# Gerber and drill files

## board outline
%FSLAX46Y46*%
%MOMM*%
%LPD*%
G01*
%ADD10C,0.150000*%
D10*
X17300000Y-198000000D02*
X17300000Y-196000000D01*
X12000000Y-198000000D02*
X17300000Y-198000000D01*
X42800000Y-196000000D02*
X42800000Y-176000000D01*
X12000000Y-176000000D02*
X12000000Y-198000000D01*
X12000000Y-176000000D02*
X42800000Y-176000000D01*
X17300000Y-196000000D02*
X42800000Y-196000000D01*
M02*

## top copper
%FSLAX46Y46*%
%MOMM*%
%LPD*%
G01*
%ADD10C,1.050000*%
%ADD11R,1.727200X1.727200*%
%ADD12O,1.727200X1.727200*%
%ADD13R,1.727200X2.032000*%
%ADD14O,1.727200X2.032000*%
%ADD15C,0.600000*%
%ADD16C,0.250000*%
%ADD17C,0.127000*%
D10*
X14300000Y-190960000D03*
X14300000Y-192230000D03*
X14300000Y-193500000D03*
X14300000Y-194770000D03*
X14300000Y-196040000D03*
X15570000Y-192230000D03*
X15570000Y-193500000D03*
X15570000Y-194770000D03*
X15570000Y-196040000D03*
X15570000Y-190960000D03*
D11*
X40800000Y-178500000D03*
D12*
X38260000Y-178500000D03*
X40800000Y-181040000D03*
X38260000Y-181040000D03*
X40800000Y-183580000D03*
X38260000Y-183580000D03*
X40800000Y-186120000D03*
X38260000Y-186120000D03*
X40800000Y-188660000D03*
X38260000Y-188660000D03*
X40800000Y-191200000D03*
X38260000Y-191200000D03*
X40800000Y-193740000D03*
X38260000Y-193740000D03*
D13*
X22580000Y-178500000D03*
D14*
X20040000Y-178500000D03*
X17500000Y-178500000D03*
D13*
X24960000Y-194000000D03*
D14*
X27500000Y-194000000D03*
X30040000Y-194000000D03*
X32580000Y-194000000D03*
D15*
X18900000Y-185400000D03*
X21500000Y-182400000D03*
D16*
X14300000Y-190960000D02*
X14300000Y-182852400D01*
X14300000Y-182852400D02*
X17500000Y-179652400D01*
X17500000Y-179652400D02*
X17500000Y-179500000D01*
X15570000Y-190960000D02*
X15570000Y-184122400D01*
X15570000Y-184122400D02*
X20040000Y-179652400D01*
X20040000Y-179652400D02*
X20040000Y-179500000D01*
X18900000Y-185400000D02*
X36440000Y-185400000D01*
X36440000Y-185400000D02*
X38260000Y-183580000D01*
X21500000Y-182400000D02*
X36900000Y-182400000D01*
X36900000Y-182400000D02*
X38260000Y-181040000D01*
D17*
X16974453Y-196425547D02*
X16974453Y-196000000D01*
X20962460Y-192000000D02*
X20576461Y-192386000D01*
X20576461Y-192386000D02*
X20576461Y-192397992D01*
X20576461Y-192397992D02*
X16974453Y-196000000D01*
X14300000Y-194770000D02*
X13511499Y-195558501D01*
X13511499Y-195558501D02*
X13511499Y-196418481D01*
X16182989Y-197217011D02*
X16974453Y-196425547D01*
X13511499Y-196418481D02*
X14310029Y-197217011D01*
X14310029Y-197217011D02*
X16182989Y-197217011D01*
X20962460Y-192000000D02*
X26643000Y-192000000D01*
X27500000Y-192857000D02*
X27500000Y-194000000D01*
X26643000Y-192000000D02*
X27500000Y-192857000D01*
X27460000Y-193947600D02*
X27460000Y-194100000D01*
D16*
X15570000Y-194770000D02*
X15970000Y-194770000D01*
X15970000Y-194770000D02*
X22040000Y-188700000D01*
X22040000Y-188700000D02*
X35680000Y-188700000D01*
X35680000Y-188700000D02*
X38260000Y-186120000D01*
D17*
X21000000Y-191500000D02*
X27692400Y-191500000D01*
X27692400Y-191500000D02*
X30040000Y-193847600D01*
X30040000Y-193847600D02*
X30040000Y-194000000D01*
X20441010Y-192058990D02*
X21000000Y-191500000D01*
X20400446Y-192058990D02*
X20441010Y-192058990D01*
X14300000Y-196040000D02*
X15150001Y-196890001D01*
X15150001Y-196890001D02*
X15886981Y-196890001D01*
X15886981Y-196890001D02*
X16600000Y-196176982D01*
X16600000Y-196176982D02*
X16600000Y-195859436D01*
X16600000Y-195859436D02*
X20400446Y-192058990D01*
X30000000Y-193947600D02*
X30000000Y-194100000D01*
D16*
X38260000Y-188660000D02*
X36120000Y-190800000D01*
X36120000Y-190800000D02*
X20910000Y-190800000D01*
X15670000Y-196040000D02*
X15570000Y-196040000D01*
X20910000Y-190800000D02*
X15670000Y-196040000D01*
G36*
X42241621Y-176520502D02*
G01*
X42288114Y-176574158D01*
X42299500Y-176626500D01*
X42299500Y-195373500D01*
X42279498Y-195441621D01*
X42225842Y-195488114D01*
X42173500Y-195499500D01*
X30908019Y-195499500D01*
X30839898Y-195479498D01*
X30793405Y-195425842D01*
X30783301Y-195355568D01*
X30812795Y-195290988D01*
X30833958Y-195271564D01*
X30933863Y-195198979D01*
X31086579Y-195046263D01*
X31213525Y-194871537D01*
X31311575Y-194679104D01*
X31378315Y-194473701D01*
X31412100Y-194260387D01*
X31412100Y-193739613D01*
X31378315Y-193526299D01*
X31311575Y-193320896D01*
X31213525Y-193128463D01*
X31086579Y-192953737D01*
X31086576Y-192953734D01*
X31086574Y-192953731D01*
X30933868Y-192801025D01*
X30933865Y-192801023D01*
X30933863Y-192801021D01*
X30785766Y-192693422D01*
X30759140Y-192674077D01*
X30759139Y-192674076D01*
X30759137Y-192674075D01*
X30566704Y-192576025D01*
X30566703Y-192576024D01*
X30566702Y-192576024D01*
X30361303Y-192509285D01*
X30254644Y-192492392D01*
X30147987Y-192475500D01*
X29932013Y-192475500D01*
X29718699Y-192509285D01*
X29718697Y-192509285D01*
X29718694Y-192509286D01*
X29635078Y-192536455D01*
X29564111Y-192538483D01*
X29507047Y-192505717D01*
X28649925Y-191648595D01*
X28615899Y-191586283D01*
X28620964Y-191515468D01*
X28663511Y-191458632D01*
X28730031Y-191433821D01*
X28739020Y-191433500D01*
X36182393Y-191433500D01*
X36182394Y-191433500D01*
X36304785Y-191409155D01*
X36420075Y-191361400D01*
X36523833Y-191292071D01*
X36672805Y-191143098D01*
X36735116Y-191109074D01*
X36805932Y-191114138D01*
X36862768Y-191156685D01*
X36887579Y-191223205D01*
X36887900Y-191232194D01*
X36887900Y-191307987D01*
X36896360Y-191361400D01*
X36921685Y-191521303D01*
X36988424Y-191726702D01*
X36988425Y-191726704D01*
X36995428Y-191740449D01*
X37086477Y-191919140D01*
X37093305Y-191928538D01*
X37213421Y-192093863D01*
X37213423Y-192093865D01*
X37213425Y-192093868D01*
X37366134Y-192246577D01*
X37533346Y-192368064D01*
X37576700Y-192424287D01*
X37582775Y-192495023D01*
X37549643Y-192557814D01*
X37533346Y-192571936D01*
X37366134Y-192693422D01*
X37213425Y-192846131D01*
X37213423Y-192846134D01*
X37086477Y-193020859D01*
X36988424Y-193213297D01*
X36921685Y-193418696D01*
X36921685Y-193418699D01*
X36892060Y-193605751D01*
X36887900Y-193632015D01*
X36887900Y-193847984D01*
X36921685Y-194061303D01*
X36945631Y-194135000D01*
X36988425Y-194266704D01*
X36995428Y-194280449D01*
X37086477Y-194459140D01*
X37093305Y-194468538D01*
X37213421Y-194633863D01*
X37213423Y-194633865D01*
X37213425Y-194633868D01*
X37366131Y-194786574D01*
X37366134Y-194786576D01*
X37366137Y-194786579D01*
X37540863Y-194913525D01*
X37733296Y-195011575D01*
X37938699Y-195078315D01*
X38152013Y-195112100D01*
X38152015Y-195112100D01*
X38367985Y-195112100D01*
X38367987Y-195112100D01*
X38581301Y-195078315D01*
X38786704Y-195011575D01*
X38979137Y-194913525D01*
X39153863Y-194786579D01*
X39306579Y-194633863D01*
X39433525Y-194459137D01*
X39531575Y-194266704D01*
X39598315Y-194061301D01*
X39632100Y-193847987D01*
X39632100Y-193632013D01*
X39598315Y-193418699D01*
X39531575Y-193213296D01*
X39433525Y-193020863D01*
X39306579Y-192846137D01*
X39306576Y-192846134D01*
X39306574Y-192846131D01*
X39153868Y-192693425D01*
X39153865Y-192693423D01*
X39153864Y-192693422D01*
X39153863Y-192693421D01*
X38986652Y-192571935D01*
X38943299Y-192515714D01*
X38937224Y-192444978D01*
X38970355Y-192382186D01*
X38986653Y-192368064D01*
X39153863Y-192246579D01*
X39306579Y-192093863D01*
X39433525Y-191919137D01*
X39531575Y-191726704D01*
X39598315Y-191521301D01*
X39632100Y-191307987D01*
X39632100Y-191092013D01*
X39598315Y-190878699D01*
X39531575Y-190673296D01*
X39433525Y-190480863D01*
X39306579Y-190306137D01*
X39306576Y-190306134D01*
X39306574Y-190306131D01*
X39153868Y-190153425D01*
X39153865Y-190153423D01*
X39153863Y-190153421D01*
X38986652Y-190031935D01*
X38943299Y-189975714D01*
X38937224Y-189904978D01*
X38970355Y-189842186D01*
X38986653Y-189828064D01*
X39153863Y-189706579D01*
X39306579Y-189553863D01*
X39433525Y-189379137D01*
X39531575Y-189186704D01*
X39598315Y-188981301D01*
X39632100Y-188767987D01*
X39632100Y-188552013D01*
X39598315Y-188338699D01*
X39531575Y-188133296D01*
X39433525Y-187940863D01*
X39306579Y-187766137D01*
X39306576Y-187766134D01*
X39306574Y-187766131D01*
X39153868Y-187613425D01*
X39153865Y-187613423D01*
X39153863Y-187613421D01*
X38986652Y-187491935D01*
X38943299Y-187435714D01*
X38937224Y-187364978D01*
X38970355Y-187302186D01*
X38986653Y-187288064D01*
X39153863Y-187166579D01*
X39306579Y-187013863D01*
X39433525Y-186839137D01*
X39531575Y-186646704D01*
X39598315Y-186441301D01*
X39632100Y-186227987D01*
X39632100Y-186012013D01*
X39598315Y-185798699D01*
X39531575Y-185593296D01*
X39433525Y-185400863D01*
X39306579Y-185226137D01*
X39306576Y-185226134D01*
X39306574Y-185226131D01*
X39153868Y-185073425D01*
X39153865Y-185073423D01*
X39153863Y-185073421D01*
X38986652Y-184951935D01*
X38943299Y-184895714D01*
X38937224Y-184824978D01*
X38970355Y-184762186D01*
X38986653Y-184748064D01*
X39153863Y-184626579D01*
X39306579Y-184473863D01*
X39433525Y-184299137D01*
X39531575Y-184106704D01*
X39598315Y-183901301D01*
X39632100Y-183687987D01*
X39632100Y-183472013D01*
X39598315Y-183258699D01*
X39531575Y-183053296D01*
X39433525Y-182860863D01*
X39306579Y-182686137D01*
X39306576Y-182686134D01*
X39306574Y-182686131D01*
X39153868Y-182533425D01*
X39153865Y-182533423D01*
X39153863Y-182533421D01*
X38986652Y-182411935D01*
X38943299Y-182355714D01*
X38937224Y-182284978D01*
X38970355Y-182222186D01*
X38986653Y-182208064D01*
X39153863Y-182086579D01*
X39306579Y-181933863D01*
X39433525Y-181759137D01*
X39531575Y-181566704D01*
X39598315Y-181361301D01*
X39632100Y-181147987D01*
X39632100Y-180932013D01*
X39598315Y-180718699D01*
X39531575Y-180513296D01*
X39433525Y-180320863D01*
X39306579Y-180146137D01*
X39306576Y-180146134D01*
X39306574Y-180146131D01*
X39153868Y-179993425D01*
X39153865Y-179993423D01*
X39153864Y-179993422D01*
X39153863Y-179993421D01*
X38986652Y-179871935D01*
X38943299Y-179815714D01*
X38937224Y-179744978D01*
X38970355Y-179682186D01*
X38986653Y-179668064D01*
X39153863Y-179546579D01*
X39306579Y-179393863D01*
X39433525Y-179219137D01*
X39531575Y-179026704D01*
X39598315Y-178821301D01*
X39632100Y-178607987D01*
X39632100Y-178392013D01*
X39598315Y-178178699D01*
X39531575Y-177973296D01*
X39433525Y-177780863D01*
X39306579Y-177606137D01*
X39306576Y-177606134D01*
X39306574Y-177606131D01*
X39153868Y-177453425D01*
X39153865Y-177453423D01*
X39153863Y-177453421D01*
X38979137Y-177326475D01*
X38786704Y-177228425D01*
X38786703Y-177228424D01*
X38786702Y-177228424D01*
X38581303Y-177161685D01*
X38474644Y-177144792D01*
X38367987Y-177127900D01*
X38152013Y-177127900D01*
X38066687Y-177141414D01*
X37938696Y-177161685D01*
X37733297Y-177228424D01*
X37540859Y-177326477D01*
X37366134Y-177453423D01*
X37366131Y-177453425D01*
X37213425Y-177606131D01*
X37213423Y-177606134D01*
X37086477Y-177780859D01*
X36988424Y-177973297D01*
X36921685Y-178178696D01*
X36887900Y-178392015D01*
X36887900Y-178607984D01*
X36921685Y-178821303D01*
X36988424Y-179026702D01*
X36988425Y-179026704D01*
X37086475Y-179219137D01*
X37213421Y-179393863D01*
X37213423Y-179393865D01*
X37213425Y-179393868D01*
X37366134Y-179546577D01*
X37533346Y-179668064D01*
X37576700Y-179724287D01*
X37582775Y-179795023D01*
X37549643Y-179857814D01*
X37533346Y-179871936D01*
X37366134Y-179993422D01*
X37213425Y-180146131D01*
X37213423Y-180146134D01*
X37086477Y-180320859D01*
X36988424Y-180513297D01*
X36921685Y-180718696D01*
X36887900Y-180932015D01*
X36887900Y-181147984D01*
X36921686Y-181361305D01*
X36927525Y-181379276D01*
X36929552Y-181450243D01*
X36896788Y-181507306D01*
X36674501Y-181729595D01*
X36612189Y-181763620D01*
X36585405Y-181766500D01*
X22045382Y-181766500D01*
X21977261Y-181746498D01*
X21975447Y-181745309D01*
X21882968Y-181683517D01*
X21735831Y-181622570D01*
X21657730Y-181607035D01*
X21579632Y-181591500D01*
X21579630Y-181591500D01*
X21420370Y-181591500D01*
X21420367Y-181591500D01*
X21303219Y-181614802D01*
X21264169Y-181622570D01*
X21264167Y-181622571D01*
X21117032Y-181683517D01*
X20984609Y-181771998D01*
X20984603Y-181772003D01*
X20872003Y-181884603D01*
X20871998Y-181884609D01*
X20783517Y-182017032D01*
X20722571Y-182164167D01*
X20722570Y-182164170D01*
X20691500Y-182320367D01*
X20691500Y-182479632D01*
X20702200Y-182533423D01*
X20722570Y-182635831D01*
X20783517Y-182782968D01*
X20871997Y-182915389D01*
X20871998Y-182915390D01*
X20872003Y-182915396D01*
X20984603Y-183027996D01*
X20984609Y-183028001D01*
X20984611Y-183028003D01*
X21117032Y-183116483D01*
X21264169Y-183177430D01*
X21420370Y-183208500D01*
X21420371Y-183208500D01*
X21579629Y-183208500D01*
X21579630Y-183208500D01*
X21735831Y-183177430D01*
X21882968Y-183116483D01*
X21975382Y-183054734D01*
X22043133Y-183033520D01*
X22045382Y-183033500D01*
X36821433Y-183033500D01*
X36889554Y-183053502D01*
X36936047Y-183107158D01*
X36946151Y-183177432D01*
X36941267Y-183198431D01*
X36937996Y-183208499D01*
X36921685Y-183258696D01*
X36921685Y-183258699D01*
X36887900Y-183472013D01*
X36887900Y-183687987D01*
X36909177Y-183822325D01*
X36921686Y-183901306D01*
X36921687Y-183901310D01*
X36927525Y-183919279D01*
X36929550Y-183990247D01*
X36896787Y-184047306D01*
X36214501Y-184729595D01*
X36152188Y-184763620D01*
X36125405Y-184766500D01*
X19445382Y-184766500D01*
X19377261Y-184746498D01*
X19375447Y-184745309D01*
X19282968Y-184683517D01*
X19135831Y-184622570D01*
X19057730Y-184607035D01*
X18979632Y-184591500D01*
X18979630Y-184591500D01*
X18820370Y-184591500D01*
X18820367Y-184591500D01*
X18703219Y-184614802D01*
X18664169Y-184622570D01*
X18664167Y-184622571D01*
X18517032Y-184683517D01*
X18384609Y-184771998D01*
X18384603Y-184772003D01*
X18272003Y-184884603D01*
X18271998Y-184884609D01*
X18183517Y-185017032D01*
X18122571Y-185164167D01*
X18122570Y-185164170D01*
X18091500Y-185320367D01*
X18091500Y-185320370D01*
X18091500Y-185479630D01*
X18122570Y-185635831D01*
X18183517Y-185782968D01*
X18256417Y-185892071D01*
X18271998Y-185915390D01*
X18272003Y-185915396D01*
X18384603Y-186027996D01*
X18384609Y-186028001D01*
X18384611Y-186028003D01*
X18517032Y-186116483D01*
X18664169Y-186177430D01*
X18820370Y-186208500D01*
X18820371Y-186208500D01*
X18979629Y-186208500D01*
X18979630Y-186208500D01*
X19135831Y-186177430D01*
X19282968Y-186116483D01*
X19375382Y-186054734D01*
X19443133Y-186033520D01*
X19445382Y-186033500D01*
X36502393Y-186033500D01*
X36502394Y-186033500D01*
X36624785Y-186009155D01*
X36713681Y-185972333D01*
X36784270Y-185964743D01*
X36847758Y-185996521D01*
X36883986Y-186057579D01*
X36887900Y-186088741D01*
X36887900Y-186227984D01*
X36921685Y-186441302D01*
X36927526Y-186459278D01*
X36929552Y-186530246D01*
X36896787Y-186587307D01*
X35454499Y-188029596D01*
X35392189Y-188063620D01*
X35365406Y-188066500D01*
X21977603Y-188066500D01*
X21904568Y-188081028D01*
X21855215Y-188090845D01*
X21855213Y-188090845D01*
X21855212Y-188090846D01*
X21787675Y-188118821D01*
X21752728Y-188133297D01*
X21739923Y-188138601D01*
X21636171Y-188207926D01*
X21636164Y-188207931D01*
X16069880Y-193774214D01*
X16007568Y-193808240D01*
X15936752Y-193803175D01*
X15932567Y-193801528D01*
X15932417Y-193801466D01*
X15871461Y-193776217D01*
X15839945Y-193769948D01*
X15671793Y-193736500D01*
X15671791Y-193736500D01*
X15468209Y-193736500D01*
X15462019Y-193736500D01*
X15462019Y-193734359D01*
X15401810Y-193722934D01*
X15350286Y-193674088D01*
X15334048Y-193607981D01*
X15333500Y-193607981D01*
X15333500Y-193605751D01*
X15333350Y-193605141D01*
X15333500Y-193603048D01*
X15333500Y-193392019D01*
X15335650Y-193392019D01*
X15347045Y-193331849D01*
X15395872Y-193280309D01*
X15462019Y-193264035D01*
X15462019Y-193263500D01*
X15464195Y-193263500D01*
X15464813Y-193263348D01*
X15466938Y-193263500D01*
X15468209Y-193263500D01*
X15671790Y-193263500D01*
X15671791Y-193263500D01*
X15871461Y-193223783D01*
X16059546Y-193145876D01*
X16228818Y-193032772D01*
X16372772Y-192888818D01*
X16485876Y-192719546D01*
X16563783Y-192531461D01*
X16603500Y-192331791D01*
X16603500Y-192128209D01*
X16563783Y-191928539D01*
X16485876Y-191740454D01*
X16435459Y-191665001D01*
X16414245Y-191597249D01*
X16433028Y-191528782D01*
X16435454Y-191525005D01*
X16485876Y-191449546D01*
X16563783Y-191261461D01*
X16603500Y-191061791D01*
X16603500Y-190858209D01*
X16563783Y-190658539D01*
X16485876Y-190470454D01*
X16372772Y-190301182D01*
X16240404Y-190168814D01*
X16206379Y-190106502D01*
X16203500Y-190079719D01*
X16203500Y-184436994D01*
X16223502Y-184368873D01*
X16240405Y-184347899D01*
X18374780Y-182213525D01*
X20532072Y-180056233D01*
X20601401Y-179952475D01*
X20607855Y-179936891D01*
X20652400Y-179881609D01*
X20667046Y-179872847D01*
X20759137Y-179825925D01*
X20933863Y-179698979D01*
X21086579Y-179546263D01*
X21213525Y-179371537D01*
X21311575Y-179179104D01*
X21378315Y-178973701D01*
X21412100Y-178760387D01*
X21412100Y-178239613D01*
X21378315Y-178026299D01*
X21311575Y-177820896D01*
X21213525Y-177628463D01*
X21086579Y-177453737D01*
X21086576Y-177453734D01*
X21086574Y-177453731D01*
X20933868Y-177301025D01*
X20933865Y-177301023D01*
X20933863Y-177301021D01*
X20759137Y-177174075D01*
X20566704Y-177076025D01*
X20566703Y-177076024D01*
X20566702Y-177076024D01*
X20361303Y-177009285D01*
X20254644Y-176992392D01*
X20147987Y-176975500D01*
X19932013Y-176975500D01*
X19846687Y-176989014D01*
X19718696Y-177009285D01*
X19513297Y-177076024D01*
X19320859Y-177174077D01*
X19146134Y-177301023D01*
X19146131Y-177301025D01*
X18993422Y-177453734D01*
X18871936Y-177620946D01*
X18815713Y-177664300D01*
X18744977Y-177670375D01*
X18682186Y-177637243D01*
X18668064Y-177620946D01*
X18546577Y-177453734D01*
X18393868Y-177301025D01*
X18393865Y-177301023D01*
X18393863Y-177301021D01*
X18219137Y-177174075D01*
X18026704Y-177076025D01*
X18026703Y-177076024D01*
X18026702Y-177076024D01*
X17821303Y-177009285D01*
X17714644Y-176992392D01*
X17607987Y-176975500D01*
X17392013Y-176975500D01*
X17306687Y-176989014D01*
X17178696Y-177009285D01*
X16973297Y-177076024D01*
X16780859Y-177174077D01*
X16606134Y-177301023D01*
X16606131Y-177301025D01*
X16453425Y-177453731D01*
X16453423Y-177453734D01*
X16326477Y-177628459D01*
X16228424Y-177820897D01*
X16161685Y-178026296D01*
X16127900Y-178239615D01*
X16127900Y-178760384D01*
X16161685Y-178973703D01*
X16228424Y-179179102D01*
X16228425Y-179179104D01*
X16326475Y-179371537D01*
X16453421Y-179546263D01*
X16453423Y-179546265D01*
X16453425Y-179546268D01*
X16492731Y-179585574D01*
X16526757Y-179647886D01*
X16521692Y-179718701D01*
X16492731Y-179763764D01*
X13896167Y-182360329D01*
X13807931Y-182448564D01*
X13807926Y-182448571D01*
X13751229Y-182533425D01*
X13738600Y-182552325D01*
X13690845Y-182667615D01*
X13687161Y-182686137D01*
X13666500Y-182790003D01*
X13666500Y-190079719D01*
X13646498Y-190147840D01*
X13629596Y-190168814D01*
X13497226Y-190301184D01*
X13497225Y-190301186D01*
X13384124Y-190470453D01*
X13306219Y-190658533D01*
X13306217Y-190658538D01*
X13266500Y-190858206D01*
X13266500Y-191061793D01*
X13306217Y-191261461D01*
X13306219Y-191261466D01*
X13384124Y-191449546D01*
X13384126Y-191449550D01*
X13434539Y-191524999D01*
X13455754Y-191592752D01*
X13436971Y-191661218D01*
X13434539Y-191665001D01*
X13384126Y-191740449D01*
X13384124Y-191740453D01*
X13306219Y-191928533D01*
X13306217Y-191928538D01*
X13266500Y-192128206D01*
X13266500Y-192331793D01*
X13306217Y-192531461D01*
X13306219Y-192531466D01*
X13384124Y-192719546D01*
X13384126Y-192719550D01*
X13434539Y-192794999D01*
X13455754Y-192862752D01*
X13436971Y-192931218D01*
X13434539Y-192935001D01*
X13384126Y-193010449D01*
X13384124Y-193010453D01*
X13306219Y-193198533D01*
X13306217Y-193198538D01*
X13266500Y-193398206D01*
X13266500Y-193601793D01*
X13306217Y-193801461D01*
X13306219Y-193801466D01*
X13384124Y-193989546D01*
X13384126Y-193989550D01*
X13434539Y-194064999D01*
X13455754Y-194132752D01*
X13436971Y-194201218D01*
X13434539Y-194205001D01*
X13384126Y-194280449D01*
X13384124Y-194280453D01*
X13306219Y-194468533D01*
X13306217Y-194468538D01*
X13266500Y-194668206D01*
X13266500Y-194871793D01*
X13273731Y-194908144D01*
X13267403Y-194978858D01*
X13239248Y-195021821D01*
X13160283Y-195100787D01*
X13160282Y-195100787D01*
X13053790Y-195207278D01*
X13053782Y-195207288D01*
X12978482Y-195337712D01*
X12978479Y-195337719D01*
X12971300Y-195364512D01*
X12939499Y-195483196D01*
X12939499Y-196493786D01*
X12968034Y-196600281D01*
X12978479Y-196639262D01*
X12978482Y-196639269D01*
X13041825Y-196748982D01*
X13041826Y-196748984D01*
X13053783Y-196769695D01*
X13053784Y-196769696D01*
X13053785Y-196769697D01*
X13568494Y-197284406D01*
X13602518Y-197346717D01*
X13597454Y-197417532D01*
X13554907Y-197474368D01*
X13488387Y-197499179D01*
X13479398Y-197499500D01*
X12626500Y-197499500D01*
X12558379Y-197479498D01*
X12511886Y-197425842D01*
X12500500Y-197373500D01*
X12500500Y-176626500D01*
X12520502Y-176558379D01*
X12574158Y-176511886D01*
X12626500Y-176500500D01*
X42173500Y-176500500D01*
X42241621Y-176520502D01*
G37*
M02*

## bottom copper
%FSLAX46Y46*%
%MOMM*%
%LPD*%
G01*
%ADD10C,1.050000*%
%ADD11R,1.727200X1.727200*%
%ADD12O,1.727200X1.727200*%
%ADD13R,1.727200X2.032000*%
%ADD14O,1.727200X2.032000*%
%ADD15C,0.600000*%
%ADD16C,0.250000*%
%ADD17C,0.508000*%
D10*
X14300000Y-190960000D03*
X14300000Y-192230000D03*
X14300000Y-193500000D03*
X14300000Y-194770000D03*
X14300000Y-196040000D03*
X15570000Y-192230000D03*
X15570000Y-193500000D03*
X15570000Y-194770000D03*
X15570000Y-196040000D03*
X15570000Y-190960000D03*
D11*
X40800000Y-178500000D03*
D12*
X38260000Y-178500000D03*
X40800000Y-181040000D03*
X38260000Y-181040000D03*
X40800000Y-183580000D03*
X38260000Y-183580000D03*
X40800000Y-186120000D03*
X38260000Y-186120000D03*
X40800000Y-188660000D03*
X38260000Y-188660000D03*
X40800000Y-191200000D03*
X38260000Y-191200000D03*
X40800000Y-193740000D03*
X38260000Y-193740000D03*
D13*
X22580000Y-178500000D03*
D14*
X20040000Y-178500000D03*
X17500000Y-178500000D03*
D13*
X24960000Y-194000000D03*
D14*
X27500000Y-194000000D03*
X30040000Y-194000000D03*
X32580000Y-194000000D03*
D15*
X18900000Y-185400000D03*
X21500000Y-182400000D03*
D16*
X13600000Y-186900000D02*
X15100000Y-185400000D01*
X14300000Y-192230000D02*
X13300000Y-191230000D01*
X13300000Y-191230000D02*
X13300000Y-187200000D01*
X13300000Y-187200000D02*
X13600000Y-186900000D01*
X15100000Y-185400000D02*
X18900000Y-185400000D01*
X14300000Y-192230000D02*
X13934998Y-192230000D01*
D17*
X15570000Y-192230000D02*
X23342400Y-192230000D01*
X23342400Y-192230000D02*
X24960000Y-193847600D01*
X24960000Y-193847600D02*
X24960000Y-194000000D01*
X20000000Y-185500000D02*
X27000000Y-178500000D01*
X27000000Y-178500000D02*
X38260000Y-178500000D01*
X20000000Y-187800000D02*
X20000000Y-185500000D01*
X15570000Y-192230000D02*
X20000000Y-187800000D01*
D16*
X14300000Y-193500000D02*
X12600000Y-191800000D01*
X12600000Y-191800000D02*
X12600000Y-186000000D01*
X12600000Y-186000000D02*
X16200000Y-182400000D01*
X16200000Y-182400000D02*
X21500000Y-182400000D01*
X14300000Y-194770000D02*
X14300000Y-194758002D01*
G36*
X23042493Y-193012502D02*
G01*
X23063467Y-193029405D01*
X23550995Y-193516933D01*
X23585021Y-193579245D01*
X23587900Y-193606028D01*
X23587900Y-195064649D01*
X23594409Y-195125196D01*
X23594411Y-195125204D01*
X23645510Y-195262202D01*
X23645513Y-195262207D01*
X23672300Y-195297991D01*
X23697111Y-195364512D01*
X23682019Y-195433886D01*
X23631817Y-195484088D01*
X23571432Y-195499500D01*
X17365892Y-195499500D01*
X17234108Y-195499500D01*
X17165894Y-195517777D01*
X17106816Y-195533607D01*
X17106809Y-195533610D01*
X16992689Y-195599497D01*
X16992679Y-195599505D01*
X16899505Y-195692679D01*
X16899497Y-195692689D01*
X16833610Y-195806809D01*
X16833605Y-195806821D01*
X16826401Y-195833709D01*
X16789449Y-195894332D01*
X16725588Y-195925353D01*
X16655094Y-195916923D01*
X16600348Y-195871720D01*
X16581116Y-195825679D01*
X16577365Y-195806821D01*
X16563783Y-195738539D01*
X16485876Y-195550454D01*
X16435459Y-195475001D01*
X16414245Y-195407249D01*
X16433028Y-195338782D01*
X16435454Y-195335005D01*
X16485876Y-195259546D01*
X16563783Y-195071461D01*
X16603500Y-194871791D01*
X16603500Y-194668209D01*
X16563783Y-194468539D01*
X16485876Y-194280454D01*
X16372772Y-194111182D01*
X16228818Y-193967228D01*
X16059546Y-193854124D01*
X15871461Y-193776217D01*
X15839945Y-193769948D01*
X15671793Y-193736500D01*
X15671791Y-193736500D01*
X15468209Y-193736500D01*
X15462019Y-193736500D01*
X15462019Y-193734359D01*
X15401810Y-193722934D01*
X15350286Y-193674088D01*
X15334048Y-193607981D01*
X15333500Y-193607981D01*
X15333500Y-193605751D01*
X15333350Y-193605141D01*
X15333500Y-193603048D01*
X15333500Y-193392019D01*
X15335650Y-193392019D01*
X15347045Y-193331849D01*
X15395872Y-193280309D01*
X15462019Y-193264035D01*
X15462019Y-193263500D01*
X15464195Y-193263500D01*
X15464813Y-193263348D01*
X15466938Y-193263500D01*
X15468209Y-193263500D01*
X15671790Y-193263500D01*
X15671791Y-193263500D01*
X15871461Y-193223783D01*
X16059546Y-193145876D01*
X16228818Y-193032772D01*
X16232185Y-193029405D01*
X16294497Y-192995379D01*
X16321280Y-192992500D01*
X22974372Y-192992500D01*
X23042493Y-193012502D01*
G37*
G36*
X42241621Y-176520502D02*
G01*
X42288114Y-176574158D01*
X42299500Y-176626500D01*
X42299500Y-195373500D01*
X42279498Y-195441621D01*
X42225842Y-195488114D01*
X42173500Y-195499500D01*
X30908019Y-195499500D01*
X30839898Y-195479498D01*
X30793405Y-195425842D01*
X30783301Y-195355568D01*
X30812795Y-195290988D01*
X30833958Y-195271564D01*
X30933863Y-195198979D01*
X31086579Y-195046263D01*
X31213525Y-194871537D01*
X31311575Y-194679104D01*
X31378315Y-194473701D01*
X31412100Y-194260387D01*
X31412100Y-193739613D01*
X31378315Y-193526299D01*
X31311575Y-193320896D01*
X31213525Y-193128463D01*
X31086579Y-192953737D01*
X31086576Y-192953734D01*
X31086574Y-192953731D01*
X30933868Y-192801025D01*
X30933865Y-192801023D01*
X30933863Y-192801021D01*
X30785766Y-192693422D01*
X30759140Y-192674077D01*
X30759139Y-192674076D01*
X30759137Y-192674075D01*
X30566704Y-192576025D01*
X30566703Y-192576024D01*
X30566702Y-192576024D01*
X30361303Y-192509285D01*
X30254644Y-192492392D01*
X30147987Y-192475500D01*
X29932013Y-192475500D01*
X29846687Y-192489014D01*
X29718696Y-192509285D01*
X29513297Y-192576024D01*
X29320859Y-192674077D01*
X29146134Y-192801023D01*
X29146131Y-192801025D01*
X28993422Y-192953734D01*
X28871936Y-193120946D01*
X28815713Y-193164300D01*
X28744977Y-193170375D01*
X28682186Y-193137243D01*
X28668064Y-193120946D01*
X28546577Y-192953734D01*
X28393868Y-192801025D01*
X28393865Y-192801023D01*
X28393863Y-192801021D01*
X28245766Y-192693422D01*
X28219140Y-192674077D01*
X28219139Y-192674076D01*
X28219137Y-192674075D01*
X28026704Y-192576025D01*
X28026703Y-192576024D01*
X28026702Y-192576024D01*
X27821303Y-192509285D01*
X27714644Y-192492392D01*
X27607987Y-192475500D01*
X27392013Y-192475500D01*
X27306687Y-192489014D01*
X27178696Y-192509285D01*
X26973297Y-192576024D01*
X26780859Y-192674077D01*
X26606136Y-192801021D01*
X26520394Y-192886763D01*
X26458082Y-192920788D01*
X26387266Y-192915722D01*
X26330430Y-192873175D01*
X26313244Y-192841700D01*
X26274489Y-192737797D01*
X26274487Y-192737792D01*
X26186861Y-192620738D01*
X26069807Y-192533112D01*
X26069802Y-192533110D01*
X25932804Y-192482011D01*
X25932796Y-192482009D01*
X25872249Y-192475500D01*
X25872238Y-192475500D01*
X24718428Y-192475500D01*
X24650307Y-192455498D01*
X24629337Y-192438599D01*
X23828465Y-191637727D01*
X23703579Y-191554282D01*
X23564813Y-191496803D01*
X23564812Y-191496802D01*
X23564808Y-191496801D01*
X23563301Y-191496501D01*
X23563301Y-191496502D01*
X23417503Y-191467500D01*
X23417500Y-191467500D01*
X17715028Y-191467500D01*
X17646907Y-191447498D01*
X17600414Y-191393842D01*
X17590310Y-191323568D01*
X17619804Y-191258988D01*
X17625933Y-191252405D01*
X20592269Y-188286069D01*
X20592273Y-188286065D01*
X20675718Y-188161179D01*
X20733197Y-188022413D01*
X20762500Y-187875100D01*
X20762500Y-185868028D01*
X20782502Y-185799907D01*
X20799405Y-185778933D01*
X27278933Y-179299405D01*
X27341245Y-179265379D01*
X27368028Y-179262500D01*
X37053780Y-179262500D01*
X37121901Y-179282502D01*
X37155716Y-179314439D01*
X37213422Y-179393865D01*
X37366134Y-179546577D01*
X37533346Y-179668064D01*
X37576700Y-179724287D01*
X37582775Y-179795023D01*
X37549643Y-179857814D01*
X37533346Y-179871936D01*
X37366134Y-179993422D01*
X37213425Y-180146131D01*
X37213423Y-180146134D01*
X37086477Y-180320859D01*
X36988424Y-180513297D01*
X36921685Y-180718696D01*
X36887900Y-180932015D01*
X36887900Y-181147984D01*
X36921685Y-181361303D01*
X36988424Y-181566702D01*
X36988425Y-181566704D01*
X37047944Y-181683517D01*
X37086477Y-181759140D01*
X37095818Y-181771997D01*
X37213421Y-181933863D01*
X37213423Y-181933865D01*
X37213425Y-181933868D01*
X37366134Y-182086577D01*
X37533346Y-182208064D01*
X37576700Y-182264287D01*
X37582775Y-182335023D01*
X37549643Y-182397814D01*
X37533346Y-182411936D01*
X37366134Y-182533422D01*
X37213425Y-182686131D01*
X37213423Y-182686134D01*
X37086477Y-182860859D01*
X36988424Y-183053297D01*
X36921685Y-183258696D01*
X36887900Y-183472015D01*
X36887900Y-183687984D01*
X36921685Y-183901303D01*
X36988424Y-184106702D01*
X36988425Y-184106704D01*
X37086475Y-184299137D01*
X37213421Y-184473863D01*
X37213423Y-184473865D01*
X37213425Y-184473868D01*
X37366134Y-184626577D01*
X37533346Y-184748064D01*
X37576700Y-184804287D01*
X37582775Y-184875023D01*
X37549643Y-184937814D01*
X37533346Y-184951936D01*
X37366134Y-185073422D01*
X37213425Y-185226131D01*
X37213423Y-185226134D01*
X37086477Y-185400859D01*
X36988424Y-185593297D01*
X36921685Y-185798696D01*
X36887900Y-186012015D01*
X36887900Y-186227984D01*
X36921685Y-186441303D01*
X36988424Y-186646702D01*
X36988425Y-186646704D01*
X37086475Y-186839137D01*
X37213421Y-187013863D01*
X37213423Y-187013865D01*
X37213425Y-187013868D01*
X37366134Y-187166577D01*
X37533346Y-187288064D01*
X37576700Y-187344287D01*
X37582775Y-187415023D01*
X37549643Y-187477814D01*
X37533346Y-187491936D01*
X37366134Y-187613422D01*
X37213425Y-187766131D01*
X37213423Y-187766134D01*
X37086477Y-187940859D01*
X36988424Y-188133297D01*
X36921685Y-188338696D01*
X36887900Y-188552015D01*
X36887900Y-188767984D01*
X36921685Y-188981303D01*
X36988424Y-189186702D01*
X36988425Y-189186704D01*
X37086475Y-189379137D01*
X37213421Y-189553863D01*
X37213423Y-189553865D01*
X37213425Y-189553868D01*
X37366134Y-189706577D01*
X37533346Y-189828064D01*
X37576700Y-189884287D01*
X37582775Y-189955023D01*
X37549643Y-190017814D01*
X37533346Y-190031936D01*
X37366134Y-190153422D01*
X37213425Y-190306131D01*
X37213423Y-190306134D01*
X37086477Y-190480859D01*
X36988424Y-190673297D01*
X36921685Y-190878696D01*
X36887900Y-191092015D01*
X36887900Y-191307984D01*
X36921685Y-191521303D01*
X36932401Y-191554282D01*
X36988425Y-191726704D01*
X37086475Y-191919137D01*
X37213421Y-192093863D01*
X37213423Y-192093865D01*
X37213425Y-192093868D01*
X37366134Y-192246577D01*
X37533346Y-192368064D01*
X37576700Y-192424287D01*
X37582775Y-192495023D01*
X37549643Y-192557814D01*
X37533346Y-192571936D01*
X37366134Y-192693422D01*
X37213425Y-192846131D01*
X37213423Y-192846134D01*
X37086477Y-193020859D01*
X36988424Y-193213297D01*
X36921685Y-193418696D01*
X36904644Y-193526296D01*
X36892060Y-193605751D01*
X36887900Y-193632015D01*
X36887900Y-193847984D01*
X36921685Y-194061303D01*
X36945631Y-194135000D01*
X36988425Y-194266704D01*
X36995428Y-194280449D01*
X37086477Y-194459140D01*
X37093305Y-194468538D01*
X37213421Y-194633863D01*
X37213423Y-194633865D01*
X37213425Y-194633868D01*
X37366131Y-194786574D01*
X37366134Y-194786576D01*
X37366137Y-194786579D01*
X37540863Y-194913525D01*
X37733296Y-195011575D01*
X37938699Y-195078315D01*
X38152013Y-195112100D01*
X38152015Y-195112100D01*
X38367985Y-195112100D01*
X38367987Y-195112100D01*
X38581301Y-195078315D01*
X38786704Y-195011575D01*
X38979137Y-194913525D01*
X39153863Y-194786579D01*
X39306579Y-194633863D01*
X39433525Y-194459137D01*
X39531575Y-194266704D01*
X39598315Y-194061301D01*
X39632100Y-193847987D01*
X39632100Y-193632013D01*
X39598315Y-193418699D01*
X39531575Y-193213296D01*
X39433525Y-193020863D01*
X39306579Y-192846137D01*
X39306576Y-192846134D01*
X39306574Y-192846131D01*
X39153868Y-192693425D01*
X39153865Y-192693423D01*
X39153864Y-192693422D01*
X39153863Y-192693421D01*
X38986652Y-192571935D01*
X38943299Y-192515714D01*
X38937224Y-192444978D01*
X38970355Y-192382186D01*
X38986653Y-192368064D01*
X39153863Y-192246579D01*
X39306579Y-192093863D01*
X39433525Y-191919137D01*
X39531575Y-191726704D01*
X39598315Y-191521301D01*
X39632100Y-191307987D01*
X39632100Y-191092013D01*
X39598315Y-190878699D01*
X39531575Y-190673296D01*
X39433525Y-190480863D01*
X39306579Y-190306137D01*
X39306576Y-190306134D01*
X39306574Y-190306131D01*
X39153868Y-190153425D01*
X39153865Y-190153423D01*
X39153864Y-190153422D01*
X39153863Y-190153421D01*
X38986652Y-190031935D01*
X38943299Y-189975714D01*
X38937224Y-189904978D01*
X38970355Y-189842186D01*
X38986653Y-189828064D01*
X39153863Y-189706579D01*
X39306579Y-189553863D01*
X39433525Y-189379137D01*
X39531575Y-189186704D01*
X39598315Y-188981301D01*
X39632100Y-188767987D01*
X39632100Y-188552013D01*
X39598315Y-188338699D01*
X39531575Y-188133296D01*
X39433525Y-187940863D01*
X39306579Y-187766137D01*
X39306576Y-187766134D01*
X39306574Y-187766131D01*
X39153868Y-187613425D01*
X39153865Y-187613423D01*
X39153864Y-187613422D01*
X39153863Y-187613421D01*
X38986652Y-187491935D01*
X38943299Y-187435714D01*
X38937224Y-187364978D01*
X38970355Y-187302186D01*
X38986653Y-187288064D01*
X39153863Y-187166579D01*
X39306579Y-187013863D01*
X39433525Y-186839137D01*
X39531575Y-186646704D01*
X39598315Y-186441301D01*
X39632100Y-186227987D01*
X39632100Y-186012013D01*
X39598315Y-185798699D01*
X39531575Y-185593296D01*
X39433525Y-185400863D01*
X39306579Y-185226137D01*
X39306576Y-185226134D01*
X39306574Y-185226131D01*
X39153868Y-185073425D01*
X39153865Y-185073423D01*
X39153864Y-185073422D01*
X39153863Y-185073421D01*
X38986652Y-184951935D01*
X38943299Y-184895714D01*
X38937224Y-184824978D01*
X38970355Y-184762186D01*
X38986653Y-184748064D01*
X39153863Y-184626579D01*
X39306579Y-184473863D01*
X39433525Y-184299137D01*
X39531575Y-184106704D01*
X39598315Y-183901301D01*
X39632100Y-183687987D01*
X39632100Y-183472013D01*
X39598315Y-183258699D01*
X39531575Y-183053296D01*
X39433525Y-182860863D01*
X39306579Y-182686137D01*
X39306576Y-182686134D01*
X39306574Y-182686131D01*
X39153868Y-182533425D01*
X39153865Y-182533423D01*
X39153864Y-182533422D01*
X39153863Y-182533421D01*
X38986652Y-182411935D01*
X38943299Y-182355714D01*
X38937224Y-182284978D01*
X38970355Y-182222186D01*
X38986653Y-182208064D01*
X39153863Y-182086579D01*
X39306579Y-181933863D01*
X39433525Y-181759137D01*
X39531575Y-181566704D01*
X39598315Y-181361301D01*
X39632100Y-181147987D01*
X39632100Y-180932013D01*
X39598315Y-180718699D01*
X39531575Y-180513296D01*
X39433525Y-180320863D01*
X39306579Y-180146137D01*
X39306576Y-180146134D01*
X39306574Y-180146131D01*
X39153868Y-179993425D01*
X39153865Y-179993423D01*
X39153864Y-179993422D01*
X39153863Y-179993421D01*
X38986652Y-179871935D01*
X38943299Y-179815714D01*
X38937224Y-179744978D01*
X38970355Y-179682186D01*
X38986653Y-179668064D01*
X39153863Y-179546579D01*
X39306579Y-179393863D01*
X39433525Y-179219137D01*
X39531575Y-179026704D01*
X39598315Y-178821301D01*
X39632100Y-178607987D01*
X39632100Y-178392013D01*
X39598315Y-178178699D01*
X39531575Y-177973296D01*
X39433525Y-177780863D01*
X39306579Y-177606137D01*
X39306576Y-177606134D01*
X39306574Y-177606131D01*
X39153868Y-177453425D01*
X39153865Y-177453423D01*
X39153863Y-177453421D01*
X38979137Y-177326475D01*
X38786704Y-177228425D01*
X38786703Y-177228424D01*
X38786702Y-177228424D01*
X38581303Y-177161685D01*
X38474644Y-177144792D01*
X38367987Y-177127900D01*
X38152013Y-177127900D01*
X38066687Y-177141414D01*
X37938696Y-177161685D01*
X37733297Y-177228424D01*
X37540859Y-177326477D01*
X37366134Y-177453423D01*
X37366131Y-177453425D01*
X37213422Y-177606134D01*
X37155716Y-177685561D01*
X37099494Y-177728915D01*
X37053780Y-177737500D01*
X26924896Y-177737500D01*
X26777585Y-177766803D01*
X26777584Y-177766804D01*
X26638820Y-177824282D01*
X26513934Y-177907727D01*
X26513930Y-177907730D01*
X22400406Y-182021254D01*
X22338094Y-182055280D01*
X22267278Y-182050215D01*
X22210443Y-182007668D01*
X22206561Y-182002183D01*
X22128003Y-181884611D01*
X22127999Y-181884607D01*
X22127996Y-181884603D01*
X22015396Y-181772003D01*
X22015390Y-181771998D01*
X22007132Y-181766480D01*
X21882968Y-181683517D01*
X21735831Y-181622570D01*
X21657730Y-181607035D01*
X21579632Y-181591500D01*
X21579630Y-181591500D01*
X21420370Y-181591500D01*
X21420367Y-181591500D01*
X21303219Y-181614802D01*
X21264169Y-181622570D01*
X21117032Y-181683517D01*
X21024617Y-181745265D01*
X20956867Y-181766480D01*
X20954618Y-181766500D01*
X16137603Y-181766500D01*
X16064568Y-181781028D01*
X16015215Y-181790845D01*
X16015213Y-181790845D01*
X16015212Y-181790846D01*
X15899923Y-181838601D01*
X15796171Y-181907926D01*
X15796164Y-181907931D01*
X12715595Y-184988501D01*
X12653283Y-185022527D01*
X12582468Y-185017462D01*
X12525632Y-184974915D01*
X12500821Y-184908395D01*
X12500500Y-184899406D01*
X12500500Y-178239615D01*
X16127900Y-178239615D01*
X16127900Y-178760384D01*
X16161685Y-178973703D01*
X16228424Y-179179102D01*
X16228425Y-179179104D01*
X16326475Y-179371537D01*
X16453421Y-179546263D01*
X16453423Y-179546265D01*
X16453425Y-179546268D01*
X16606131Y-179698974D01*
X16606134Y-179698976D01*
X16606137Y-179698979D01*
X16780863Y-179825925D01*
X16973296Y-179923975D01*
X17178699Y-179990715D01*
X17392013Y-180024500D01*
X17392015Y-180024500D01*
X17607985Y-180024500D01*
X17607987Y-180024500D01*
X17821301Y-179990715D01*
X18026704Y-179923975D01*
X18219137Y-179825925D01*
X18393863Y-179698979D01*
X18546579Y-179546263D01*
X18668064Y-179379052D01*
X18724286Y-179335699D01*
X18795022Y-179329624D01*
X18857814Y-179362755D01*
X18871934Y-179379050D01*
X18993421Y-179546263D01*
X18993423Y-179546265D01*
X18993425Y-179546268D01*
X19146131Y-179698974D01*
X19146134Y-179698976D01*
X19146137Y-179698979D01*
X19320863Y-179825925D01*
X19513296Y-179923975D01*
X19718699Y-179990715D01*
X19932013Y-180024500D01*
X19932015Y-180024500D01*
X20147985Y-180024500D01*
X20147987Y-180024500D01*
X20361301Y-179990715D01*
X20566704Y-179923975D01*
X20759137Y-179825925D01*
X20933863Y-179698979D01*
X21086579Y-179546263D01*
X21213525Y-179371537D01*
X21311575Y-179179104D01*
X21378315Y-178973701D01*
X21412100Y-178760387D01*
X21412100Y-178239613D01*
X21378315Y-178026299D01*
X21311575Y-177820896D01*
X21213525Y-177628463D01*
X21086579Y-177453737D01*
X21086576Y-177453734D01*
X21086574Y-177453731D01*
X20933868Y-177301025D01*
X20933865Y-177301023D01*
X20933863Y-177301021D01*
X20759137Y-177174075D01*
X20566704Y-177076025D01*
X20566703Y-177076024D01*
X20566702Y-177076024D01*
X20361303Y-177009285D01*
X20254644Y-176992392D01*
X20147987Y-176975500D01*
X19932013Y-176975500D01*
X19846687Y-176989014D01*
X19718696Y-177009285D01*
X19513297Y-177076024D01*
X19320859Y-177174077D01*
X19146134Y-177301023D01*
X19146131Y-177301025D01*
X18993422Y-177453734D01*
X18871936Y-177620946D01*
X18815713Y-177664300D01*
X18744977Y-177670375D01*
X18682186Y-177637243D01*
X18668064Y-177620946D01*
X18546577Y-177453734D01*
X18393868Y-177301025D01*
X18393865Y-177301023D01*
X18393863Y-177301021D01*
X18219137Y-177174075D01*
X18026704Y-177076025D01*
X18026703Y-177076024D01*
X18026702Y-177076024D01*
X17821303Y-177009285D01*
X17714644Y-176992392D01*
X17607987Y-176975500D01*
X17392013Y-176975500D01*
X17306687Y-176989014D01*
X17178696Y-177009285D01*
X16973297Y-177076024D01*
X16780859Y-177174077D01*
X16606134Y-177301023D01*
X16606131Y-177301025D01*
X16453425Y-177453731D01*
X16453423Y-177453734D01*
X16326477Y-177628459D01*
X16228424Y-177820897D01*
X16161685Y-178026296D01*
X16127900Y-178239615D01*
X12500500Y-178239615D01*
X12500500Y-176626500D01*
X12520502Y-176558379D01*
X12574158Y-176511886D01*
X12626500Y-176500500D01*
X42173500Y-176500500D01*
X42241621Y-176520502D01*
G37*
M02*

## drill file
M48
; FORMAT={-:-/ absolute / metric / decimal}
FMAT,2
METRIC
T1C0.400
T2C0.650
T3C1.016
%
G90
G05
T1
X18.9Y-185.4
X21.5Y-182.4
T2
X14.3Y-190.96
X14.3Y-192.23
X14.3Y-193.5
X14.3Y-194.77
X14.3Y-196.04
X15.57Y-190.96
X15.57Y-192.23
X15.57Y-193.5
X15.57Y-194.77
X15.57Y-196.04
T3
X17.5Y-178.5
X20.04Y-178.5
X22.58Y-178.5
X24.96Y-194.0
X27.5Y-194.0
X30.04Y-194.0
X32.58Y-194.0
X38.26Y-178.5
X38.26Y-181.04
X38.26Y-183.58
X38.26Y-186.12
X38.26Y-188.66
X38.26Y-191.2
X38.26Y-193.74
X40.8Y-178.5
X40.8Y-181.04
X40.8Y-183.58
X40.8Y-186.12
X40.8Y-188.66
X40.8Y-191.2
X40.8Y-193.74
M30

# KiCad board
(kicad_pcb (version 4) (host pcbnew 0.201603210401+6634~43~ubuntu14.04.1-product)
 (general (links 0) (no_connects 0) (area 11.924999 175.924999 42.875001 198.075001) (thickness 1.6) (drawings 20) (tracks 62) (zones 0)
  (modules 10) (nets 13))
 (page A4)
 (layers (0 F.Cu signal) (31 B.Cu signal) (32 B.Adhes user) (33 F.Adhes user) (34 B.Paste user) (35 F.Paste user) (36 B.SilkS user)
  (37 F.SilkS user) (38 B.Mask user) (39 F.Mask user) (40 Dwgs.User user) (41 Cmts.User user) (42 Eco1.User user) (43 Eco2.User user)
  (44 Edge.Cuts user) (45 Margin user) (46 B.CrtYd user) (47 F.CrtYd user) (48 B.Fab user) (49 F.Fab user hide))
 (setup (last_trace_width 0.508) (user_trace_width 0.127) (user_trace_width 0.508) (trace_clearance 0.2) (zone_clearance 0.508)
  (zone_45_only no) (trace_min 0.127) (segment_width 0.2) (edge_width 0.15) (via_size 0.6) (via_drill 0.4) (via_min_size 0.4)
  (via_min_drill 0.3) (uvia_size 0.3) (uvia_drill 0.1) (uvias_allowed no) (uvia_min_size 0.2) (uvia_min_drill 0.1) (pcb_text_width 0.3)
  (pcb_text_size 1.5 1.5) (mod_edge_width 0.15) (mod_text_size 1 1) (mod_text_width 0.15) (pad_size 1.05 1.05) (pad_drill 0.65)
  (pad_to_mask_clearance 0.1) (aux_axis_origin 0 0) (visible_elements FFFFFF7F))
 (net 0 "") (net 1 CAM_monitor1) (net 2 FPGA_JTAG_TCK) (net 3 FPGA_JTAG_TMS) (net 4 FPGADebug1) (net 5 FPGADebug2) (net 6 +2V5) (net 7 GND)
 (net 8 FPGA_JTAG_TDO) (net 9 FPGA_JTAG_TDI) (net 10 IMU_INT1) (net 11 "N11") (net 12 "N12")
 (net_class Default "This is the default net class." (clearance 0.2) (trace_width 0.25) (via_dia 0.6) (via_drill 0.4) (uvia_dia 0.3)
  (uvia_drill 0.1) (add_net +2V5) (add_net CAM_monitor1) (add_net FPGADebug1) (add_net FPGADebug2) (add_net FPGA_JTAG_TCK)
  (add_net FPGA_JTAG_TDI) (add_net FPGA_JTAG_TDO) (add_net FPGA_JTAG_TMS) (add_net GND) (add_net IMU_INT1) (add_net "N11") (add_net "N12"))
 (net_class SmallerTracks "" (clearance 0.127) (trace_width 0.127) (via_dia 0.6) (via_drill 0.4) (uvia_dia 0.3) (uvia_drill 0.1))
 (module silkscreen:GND (layer B.Cu) (at 42.1 195 180)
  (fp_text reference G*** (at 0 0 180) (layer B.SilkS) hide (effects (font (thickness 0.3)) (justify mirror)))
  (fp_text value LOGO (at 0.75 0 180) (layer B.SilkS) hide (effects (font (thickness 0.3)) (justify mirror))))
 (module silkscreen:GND (layer B.Cu) (at 42.1 176.8 180)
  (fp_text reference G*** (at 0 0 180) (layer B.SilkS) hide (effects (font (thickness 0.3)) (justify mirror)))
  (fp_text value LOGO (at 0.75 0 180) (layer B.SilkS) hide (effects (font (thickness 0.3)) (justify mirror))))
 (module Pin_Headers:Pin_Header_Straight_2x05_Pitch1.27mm (layer F.Cu) (at 14.3 190.96)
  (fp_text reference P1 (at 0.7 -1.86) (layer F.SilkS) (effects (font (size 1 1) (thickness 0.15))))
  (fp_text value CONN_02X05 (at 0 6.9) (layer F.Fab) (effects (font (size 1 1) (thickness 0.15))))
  (pad 1 thru_hole circle (at 0 0) (size 1.05 1.05) (drill 0.65) (layers *.Cu *.Mask F.SilkS) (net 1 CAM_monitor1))
  (pad 3 thru_hole circle (at 0 1.27) (size 1.05 1.05) (drill 0.65) (layers *.Cu *.Mask F.SilkS) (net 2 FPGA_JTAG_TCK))
  (pad 5 thru_hole circle (at 0 2.54) (size 1.05 1.05) (drill 0.65) (layers *.Cu *.Mask F.SilkS) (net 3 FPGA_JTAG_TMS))
  (pad 7 thru_hole circle (at 0 3.81) (size 1.05 1.05) (drill 0.65) (layers *.Cu *.Mask F.SilkS) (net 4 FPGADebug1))
  (pad 9 thru_hole circle (at 0 5.08) (size 1.05 1.05) (drill 0.65) (layers *.Cu *.Mask F.SilkS) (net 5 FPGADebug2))
  (pad 4 thru_hole circle (at 1.27 1.27) (size 1.05 1.05) (drill 0.65) (layers *.Cu *.Mask F.SilkS) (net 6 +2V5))
  (pad 6 thru_hole circle (at 1.27 2.54) (size 1.05 1.05) (drill 0.65) (layers *.Cu *.Mask F.SilkS) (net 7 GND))
  (pad 8 thru_hole circle (at 1.27 3.81) (size 1.05 1.05) (drill 0.65) (layers *.Cu *.Mask F.SilkS) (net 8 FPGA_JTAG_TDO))
  (pad 10 thru_hole circle (at 1.27 5.08) (size 1.05 1.05) (drill 0.65) (layers *.Cu *.Mask F.SilkS) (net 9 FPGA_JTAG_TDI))
  (pad 2 thru_hole circle (at 1.27 0) (size 1.05 1.05) (drill 0.65) (layers *.Cu *.Mask F.SilkS) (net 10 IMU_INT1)))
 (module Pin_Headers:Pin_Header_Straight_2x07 (layer B.Cu) (at 40.8 178.5 180)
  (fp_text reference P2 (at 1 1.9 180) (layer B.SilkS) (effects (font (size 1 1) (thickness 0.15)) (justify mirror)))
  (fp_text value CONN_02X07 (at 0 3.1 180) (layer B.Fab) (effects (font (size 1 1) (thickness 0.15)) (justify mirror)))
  (pad 1 thru_hole rect (at 0 0 180) (size 1.7272 1.7272) (drill 1.016) (layers *.Cu *.Mask B.SilkS) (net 7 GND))
  (pad 2 thru_hole oval (at 2.54 0 180) (size 1.7272 1.7272) (drill 1.016) (layers *.Cu *.Mask B.SilkS) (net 6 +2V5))
  (pad 3 thru_hole oval (at 0 -2.54 180) (size 1.7272 1.7272) (drill 1.016) (layers *.Cu *.Mask B.SilkS) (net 7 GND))
  (pad 4 thru_hole oval (at 2.54 -2.54 180) (size 1.7272 1.7272) (drill 1.016) (layers *.Cu *.Mask B.SilkS) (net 3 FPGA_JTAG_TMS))
  (pad 5 thru_hole oval (at 0 -5.08 180) (size 1.7272 1.7272) (drill 1.016) (layers *.Cu *.Mask B.SilkS) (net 7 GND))
  (pad 6 thru_hole oval (at 2.54 -5.08 180) (size 1.7272 1.7272) (drill 1.016) (layers *.Cu *.Mask B.SilkS) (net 2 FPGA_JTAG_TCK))
  (pad 7 thru_hole oval (at 0 -7.62 180) (size 1.7272 1.7272) (drill 1.016) (layers *.Cu *.Mask B.SilkS) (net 7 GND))
  (pad 8 thru_hole oval (at 2.54 -7.62 180) (size 1.7272 1.7272) (drill 1.016) (layers *.Cu *.Mask B.SilkS) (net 8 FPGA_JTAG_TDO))
  (pad 9 thru_hole oval (at 0 -10.16 180) (size 1.7272 1.7272) (drill 1.016) (layers *.Cu *.Mask B.SilkS) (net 7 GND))
  (pad 10 thru_hole oval (at 2.54 -10.16 180) (size 1.7272 1.7272) (drill 1.016) (layers *.Cu *.Mask B.SilkS) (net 9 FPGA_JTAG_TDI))
  (pad 11 thru_hole oval (at 0 -12.7 180) (size 1.7272 1.7272) (drill 1.016) (layers *.Cu *.Mask B.SilkS) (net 7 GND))
  (pad 12 thru_hole oval (at 2.54 -12.7 180) (size 1.7272 1.7272) (drill 1.016) (layers *.Cu *.Mask B.SilkS) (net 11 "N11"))
  (pad 13 thru_hole oval (at 0 -15.24 180) (size 1.7272 1.7272) (drill 1.016) (layers *.Cu *.Mask B.SilkS) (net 7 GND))
  (pad 14 thru_hole oval (at 2.54 -15.24 180) (size 1.7272 1.7272) (drill 1.016) (layers *.Cu *.Mask B.SilkS) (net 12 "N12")))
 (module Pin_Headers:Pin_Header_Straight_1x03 (layer B.Cu) (at 22.58 178.5 90)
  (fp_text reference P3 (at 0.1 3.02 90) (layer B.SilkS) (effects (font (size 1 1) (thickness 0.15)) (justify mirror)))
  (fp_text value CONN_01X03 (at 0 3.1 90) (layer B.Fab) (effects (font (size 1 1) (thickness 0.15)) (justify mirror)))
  (pad 1 thru_hole rect (at 0 0 90) (size 2.032 1.7272) (drill 1.016) (layers *.Cu *.Mask B.SilkS) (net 7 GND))
  (pad 2 thru_hole oval (at 0 -2.54 90) (size 2.032 1.7272) (drill 1.016) (layers *.Cu *.Mask B.SilkS) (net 10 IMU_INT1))
  (pad 3 thru_hole oval (at 0 -5.08 90) (size 2.032 1.7272) (drill 1.016) (layers *.Cu *.Mask B.SilkS) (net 1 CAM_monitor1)))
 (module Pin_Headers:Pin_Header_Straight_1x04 (layer B.Cu) (at 24.96 194 270)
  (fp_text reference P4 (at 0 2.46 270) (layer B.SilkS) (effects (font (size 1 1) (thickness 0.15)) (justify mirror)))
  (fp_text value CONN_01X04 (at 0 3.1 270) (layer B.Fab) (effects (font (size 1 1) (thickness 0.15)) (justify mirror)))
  (pad 1 thru_hole rect (at 0 0 270) (size 2.032 1.7272) (drill 1.016) (layers *.Cu *.Mask B.SilkS) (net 6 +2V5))
  (pad 2 thru_hole oval (at 0 -2.54 270) (size 2.032 1.7272) (drill 1.016) (layers *.Cu *.Mask B.SilkS) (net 4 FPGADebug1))
  (pad 3 thru_hole oval (at 0 -5.08 270) (size 2.032 1.7272) (drill 1.016) (layers *.Cu *.Mask B.SilkS) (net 5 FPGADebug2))
  (pad 4 thru_hole oval (at 0 -7.62 270) (size 2.032 1.7272) (drill 1.016) (layers *.Cu *.Mask B.SilkS) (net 7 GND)))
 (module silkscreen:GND (layer B.Cu) (at 34.8 194 180)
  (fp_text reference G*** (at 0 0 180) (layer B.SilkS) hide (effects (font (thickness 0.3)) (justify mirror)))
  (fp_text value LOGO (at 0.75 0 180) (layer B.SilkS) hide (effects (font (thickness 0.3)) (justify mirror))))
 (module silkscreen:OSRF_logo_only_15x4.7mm (layer F.Cu) (at 28.8 183.4)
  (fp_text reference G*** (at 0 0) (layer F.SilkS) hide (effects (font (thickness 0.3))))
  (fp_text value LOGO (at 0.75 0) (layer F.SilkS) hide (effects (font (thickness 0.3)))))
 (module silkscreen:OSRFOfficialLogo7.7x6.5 (layer F.Cu) (at 20.3 191.2)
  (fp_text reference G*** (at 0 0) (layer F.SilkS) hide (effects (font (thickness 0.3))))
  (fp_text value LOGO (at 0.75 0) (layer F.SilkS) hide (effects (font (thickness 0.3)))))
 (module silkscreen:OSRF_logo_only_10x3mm (layer B.Cu) (at 14 184.2 270)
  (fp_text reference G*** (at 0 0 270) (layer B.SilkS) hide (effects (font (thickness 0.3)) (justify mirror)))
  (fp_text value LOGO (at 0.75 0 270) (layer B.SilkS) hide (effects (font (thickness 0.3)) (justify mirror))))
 (gr_line (start 17.3 198) (end 17.3 196) (layer Edge.Cuts) (width 0.15))
 (gr_line (start 12 198) (end 17.3 198) (layer Edge.Cuts) (width 0.15))
 (gr_line (start 42.8 196) (end 42.8 176) (layer Edge.Cuts) (width 0.15))
 (gr_line (start 12 176) (end 12 198) (layer Edge.Cuts) (width 0.15))
 (gr_line (start 12 176) (end 42.8 176) (layer Edge.Cuts) (width 0.15))
 (gr_line (start 17.3 196) (end 42.8 196) (layer Edge.Cuts) (width 0.15))
 (segment (start 14.3 190.96) (end 14.3 182.8524) (width 0.25) (layer F.Cu) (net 1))
 (segment (start 14.3 182.8524) (end 17.5 179.6524) (width 0.25) (layer F.Cu) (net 1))
 (segment (start 17.5 179.6524) (end 17.5 179.5) (width 0.25) (layer F.Cu) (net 1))
 (segment (start 15.57 190.96) (end 15.57 184.1224) (width 0.25) (layer F.Cu) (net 10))
 (segment (start 15.57 184.1224) (end 20.04 179.6524) (width 0.25) (layer F.Cu) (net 10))
 (segment (start 20.04 179.6524) (end 20.04 179.5) (width 0.25) (layer F.Cu) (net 10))
 (segment (start 13.6 186.9) (end 15.1 185.4) (width 0.25) (layer B.Cu) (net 2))
 (segment (start 14.3 192.23) (end 13.3 191.23) (width 0.25) (layer B.Cu) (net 2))
 (segment (start 13.3 191.23) (end 13.3 187.2) (width 0.25) (layer B.Cu) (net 2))
 (segment (start 13.3 187.2) (end 13.6 186.9) (width 0.25) (layer B.Cu) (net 2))
 (segment (start 18.9 185.4) (end 36.44 185.4) (width 0.25) (layer F.Cu) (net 2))
 (segment (start 36.44 185.4) (end 38.26 183.58) (width 0.25) (layer F.Cu) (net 2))
 (segment (start 15.1 185.4) (end 18.9 185.4) (width 0.25) (layer B.Cu) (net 2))
 (via (at 18.9 185.4) (size 0.6) (drill 0.4) (layers F.Cu B.Cu) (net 2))
 (segment (start 14.3 192.23) (end 13.934998 192.23) (width 0.25) (layer B.Cu) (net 2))
 (segment (start 15.57 192.23) (end 23.3424 192.23) (width 0.508) (layer B.Cu) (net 6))
 (segment (start 23.3424 192.23) (end 24.96 193.8476) (width 0.508) (layer B.Cu) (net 6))
 (segment (start 24.96 193.8476) (end 24.96 194) (width 0.508) (layer B.Cu) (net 6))
 (segment (start 20 185.5) (end 27 178.5) (width 0.508) (layer B.Cu) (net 6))
 (segment (start 27 178.5) (end 38.26 178.5) (width 0.508) (layer B.Cu) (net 6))
 (segment (start 20 187.8) (end 20 185.5) (width 0.508) (layer B.Cu) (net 6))
 (segment (start 15.57 192.23) (end 20 187.8) (width 0.508) (layer B.Cu) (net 6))
 (segment (start 14.3 193.5) (end 12.6 191.8) (width 0.25) (layer B.Cu) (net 3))
 (segment (start 12.6 191.8) (end 12.6 186) (width 0.25) (layer B.Cu) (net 3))
 (segment (start 12.6 186) (end 16.2 182.4) (width 0.25) (layer B.Cu) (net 3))
 (segment (start 16.2 182.4) (end 21.5 182.4) (width 0.25) (layer B.Cu) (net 3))
 (segment (start 21.5 182.4) (end 36.9 182.4) (width 0.25) (layer F.Cu) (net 3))
 (segment (start 36.9 182.4) (end 38.26 181.04) (width 0.25) (layer F.Cu) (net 3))
 (via (at 21.5 182.4) (size 0.6) (drill 0.4) (layers F.Cu B.Cu) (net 3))
 (segment (start 16.974453 196.425547) (end 16.974453 196) (width 0.127) (layer F.Cu) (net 4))
 (segment (start 20.96246 192) (end 20.576461 192.386) (width 0.127) (layer F.Cu) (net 4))
 (segment (start 20.576461 192.386) (end 20.576461 192.397992) (width 0.127) (layer F.Cu) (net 4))
 (segment (start 20.576461 192.397992) (end 16.974453 196) (width 0.127) (layer F.Cu) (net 4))
 (segment (start 14.3 194.77) (end 13.511499 195.558501) (width 0.127) (layer F.Cu) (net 4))
 (segment (start 13.511499 195.558501) (end 13.511499 196.418481) (width 0.127) (layer F.Cu) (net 4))
 (segment (start 16.182989 197.217011) (end 16.974453 196.425547) (width 0.127) (layer F.Cu) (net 4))
 (segment (start 13.511499 196.418481) (end 14.310029 197.217011) (width 0.127) (layer F.Cu) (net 4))
 (segment (start 14.310029 197.217011) (end 16.182989 197.217011) (width 0.127) (layer F.Cu) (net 4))
 (segment (start 20.96246 192) (end 26.643 192) (width 0.127) (layer F.Cu) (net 4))
 (segment (start 27.5 192.857) (end 27.5 194) (width 0.127) (layer F.Cu) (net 4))
 (segment (start 26.643 192) (end 27.5 192.857) (width 0.127) (layer F.Cu) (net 4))
 (segment (start 27.46 193.9476) (end 27.46 194.1) (width 0.127) (layer F.Cu) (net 4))
 (segment (start 14.3 194.77) (end 14.3 194.758002) (width 0.25) (layer B.Cu) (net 4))
 (segment (start 15.57 194.77) (end 15.97 194.77) (width 0.25) (layer F.Cu) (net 8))
 (segment (start 15.97 194.77) (end 22.04 188.7) (width 0.25) (layer F.Cu) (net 8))
 (segment (start 22.04 188.7) (end 35.68 188.7) (width 0.25) (layer F.Cu) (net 8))
 (segment (start 35.68 188.7) (end 38.26 186.12) (width 0.25) (layer F.Cu) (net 8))
 (segment (start 21 191.5) (end 27.6924 191.5) (width 0.127) (layer F.Cu) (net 5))
 (segment (start 27.6924 191.5) (end 30.04 193.8476) (width 0.127) (layer F.Cu) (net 5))
 (segment (start 30.04 193.8476) (end 30.04 194) (width 0.127) (layer F.Cu) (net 5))
 (segment (start 20.44101 192.05899) (end 21 191.5) (width 0.127) (layer F.Cu) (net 5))
 (segment (start 20.400446 192.05899) (end 20.44101 192.05899) (width 0.127) (layer F.Cu) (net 5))
 (segment (start 14.3 196.04) (end 15.150001 196.890001) (width 0.127) (layer F.Cu) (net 5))
 (segment (start 15.150001 196.890001) (end 15.886981 196.890001) (width 0.127) (layer F.Cu) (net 5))
 (segment (start 15.886981 196.890001) (end 16.6 196.176982) (width 0.127) (layer F.Cu) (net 5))
 (segment (start 16.6 196.176982) (end 16.6 195.859436) (width 0.127) (layer F.Cu) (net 5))
 (segment (start 16.6 195.859436) (end 20.400446 192.05899) (width 0.127) (layer F.Cu) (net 5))
 (segment (start 30 193.9476) (end 30 194.1) (width 0.127) (layer F.Cu) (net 5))
 (segment (start 38.26 188.66) (end 36.12 190.8) (width 0.25) (layer F.Cu) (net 9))
 (segment (start 36.12 190.8) (end 20.91 190.8) (width 0.25) (layer F.Cu) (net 9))
 (segment (start 15.67 196.04) (end 15.57 196.04) (width 0.25) (layer F.Cu) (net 9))
 (segment (start 20.91 190.8) (end 15.67 196.04) (width 0.25) (layer F.Cu) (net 9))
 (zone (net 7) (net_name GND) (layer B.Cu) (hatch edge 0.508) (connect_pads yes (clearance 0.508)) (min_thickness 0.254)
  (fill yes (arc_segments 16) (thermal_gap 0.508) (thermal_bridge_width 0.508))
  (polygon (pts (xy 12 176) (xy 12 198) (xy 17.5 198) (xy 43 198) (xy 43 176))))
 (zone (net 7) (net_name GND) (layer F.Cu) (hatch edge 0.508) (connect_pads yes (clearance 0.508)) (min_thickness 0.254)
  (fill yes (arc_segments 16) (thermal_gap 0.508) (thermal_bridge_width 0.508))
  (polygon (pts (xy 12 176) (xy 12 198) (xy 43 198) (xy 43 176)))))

